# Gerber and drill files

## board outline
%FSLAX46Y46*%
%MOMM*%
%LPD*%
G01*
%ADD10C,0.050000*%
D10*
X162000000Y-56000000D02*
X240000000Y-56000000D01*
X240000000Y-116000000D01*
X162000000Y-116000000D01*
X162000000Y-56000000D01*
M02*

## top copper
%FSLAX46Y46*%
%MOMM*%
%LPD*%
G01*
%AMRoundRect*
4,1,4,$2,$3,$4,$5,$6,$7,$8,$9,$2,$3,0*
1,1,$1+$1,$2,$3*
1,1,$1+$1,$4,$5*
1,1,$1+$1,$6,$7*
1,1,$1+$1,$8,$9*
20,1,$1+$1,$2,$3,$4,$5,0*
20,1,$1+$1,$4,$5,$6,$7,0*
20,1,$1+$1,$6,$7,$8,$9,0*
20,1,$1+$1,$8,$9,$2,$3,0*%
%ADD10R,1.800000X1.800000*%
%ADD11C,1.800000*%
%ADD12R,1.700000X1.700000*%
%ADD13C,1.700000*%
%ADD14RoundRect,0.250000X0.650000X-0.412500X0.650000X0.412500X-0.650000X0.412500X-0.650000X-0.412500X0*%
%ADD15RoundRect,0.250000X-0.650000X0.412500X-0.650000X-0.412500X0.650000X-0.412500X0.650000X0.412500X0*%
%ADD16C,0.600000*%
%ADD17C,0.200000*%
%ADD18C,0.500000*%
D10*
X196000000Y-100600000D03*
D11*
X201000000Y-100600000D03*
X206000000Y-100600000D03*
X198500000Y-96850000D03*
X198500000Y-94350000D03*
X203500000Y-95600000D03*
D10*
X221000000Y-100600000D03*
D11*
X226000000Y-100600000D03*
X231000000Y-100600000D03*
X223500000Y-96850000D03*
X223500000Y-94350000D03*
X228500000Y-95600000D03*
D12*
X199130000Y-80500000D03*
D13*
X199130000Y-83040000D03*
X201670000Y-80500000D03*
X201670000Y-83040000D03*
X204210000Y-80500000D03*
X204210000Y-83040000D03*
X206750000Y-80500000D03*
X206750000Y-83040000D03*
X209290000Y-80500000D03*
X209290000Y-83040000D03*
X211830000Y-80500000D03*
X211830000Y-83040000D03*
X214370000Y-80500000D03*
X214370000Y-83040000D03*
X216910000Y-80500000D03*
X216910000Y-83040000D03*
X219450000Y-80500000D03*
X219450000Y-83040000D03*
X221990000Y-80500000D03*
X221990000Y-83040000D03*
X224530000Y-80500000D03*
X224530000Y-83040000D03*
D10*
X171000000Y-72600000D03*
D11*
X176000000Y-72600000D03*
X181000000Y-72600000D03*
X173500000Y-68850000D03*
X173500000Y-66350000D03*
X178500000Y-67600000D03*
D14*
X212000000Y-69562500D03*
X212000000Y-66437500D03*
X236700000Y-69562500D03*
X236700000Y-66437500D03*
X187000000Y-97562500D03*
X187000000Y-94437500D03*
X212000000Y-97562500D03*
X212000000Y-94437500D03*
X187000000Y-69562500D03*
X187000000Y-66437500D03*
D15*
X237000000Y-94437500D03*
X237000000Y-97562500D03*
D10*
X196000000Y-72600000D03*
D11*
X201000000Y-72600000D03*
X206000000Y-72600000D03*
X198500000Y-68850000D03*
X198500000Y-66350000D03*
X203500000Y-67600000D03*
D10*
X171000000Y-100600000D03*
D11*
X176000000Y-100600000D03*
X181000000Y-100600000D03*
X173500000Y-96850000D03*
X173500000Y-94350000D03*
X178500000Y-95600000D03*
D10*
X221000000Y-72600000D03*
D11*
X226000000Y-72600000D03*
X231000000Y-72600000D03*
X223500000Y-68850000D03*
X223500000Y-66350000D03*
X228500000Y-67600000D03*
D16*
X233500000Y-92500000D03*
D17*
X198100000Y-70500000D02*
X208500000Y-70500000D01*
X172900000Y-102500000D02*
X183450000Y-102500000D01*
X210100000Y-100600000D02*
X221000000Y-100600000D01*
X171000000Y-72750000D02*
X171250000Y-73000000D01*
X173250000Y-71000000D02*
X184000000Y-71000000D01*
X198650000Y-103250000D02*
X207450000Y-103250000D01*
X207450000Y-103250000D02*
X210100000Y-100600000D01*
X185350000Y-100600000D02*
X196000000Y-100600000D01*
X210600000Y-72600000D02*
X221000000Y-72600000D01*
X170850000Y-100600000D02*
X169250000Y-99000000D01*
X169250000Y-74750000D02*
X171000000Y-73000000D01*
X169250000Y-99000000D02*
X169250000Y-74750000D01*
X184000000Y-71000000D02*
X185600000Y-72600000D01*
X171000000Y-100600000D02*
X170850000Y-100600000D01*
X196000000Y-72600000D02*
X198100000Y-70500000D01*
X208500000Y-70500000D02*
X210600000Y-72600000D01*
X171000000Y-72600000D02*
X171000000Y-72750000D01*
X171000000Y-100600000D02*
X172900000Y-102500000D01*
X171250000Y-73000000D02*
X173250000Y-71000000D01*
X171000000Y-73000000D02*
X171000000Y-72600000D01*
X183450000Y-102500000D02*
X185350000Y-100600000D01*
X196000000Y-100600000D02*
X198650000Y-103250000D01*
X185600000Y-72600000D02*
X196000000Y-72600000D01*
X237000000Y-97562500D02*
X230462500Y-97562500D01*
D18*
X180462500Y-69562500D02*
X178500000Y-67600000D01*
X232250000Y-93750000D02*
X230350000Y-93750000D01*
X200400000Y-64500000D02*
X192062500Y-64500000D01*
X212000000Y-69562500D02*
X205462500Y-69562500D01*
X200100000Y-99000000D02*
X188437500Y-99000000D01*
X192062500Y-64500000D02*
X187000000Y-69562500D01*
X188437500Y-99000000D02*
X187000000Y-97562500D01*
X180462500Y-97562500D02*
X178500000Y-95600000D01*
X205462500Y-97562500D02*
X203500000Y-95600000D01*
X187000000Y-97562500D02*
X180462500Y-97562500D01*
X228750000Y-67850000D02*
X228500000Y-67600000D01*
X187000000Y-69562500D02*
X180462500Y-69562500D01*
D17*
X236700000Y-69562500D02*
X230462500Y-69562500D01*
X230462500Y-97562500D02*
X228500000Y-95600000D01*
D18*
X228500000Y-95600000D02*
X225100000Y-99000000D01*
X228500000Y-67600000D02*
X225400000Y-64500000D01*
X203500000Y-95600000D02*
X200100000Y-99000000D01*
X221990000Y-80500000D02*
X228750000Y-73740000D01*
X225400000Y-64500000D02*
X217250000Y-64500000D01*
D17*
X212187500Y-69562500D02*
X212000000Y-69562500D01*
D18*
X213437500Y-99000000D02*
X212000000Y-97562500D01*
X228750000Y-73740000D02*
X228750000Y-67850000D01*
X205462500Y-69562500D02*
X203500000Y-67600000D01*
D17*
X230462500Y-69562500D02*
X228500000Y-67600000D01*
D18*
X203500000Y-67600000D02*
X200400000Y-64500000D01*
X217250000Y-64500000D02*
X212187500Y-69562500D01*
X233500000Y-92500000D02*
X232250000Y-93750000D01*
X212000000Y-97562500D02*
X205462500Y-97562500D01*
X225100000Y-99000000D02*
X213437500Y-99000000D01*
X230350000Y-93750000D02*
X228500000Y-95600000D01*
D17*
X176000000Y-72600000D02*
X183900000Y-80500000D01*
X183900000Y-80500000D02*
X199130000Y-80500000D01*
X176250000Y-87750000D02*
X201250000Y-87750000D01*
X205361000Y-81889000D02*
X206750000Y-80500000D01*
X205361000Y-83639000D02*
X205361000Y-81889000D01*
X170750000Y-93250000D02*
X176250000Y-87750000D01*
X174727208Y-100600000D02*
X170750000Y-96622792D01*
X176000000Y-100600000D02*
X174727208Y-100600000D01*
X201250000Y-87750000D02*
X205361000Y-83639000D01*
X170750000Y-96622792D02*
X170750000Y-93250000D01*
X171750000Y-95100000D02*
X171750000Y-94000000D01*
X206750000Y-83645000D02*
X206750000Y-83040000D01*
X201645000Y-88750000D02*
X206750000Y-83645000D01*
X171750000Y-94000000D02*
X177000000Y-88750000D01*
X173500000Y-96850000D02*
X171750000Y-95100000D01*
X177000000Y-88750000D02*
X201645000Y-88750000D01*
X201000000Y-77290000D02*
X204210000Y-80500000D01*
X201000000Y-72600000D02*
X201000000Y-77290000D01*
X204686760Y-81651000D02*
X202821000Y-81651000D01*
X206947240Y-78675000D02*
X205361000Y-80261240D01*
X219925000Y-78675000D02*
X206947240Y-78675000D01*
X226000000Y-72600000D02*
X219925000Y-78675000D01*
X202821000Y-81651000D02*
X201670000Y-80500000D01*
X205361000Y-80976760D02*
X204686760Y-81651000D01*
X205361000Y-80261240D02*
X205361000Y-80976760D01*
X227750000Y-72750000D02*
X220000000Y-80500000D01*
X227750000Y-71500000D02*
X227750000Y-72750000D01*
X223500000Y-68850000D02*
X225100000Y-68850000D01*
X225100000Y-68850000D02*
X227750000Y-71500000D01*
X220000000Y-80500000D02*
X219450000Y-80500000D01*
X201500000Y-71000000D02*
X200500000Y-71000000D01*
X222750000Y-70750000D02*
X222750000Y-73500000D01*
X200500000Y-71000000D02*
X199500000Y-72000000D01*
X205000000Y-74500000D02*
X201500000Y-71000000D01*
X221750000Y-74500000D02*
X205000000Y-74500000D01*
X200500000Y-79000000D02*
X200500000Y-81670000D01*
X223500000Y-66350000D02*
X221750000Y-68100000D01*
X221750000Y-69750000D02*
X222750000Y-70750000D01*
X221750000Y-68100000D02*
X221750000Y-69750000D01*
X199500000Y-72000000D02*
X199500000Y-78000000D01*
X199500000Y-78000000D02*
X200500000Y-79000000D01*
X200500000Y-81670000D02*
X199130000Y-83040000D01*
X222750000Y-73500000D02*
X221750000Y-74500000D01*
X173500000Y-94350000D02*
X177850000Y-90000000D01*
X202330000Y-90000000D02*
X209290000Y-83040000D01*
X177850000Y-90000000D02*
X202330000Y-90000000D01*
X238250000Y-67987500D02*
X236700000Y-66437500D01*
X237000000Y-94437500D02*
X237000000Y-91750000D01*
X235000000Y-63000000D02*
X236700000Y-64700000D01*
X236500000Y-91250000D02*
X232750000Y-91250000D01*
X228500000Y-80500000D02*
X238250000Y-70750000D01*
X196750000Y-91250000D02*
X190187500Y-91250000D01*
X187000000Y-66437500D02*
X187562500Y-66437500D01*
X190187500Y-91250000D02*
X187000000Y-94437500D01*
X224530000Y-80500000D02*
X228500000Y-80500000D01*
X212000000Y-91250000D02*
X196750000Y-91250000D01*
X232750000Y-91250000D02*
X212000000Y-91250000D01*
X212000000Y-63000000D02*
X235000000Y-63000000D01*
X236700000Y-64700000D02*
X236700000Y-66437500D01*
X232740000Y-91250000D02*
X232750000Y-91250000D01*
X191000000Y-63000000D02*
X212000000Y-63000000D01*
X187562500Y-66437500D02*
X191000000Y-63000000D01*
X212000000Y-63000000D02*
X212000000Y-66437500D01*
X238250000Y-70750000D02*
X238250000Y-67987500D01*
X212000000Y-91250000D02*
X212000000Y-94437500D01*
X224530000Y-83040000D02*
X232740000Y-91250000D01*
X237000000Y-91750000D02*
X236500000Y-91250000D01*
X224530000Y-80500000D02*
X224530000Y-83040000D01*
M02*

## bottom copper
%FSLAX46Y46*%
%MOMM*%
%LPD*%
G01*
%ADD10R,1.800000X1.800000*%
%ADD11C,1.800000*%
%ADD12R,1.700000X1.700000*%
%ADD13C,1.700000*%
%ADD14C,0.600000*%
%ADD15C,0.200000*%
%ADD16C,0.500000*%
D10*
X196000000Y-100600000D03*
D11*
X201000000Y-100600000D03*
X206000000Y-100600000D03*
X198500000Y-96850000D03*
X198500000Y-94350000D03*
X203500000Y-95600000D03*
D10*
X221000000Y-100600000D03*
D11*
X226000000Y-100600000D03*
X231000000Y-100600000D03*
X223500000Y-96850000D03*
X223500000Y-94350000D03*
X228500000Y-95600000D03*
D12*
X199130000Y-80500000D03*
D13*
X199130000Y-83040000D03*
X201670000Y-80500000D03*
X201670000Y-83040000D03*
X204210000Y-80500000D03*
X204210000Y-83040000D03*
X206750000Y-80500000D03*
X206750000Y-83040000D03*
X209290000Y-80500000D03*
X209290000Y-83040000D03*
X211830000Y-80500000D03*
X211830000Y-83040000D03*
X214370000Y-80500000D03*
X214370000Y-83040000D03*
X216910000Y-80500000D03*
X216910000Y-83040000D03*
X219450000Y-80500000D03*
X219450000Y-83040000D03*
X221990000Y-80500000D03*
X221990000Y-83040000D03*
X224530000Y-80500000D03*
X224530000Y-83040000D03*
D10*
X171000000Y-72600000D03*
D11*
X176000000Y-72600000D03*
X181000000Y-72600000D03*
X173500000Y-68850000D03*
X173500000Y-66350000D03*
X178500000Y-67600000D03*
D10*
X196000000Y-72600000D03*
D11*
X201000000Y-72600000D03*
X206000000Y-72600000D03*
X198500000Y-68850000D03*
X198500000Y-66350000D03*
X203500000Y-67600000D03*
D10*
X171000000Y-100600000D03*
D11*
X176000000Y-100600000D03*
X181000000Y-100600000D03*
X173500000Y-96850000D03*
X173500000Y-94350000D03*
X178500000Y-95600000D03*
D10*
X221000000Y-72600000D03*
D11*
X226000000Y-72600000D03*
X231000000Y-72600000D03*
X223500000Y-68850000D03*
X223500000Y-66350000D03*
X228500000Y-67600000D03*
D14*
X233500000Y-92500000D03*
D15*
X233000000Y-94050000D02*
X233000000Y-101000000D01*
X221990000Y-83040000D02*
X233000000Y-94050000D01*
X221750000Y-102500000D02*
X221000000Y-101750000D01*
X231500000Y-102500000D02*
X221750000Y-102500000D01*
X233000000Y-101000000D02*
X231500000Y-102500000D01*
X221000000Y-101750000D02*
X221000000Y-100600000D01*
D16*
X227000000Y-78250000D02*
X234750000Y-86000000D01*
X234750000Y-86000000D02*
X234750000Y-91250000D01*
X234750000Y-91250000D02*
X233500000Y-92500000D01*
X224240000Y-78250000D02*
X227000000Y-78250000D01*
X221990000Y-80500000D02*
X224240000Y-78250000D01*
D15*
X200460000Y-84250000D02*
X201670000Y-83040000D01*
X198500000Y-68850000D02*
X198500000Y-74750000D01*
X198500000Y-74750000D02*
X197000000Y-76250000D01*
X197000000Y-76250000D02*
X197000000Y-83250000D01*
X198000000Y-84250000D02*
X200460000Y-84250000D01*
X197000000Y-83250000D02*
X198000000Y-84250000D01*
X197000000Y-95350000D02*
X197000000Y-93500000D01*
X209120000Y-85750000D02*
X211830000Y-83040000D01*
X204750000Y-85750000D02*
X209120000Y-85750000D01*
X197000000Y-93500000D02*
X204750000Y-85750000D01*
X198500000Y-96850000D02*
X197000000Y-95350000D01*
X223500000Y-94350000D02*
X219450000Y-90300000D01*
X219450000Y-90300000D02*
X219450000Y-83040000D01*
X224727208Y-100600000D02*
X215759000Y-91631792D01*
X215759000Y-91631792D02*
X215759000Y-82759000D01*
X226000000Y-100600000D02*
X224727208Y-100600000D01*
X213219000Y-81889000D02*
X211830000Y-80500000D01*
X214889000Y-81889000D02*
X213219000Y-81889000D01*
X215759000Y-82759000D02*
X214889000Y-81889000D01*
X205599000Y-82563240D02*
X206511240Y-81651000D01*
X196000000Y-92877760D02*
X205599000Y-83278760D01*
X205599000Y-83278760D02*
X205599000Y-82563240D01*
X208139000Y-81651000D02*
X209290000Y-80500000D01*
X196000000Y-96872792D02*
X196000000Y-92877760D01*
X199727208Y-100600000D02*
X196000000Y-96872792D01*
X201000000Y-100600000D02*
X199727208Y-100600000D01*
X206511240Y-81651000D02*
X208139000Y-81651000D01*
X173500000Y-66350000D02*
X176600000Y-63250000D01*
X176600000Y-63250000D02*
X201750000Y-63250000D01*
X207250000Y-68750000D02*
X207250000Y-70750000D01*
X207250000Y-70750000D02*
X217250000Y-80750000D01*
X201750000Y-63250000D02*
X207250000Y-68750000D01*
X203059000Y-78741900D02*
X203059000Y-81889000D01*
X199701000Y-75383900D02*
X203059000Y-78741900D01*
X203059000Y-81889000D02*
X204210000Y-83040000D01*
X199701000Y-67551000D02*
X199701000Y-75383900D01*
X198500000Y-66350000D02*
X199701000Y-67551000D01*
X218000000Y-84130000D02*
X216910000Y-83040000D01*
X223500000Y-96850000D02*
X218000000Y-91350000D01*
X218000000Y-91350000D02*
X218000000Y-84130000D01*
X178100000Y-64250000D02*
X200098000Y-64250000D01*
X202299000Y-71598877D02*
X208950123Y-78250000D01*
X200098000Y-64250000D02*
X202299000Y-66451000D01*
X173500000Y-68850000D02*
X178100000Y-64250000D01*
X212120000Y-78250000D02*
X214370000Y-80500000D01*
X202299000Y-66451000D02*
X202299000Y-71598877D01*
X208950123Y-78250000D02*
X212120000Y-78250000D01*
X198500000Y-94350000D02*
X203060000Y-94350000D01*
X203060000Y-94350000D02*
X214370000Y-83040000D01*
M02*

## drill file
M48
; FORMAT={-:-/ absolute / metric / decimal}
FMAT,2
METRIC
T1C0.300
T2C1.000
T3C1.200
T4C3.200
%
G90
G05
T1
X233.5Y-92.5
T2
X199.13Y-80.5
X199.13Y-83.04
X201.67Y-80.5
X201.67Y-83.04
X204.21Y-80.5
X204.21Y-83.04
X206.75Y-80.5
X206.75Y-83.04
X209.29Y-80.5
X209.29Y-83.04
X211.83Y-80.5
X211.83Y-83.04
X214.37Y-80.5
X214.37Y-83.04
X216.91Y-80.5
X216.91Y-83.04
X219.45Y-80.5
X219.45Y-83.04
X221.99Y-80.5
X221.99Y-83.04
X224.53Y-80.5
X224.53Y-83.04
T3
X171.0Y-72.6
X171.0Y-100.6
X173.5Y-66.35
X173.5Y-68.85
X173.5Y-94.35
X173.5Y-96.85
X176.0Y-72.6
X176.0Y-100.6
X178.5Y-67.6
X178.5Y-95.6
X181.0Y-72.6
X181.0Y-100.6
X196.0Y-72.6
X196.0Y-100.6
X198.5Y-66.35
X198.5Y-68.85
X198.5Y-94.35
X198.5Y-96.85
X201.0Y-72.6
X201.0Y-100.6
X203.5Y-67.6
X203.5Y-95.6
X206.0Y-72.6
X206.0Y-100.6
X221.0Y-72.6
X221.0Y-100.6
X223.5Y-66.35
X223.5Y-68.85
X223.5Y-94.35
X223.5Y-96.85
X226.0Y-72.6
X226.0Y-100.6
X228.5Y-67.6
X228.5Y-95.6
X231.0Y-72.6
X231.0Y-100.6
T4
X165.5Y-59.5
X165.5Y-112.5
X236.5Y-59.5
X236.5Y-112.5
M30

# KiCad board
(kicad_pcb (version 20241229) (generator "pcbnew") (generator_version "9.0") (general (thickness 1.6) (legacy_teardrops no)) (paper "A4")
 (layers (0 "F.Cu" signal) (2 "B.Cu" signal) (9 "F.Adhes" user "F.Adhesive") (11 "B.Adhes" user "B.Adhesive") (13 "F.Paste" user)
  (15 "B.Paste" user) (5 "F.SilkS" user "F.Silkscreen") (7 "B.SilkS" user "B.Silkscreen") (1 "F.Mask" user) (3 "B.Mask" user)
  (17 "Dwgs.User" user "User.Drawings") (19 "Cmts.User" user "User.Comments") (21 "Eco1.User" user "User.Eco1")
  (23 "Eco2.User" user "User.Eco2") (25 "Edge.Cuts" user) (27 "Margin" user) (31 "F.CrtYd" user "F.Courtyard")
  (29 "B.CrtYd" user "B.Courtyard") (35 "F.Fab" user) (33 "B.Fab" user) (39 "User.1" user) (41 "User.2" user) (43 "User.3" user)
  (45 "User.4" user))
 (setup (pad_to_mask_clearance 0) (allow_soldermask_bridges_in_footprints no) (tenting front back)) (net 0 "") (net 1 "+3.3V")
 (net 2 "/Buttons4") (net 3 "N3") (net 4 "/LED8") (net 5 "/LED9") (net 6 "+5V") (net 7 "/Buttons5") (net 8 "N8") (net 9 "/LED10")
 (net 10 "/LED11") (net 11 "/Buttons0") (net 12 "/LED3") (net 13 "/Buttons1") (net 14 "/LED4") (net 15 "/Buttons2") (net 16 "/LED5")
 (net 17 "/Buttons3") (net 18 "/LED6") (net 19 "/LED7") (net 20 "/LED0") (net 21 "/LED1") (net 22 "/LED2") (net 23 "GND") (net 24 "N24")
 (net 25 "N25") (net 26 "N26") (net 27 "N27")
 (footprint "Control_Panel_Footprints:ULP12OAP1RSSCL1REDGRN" (layer "F.Cu") (at 196 100.6)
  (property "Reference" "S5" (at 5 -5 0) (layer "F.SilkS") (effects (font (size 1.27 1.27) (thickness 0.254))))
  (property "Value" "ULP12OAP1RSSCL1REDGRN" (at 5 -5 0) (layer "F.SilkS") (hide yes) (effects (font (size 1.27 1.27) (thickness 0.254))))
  (pad "1" thru_hole rect (at 0 0) (size 1.8 1.8) (drill 1.2) (layers "*.Cu" "*.Mask") (remove_unused_layers no) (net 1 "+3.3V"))
  (pad "2" thru_hole circle (at 5 0) (size 1.8 1.8) (drill 1.2) (layers "*.Cu" "*.Mask") (remove_unused_layers no) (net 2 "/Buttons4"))
  (pad "3" thru_hole circle (at 10 0) (size 1.8 1.8) (drill 1.2) (layers "*.Cu" "*.Mask") (remove_unused_layers no) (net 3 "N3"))
  (pad "L1" thru_hole circle (at 2.5 -3.75) (size 1.8 1.8) (drill 1.2) (layers "*.Cu" "*.Mask") (remove_unused_layers no) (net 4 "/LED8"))
  (pad "L2" thru_hole circle (at 2.5 -6.25) (size 1.8 1.8) (drill 1.2) (layers "*.Cu" "*.Mask") (remove_unused_layers no) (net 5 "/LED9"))
  (pad "LC1" thru_hole circle (at 7.5 -5) (size 1.8 1.8) (drill 1.2) (layers "*.Cu" "*.Mask") (remove_unused_layers no) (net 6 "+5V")))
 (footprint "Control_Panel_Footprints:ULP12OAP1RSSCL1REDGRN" (layer "F.Cu") (at 221 100.6)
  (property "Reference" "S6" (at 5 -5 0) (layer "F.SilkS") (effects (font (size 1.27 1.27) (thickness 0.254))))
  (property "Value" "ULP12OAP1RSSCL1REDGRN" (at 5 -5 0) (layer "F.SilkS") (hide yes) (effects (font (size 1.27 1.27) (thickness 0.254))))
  (pad "1" thru_hole rect (at 0 0) (size 1.8 1.8) (drill 1.2) (layers "*.Cu" "*.Mask") (remove_unused_layers no) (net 1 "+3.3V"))
  (pad "2" thru_hole circle (at 5 0) (size 1.8 1.8) (drill 1.2) (layers "*.Cu" "*.Mask") (remove_unused_layers no) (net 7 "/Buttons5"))
  (pad "3" thru_hole circle (at 10 0) (size 1.8 1.8) (drill 1.2) (layers "*.Cu" "*.Mask") (remove_unused_layers no) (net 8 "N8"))
  (pad "L1" thru_hole circle (at 2.5 -3.75) (size 1.8 1.8) (drill 1.2) (layers "*.Cu" "*.Mask") (remove_unused_layers no) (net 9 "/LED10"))
  (pad "L2" thru_hole circle (at 2.5 -6.25) (size 1.8 1.8) (drill 1.2) (layers "*.Cu" "*.Mask") (remove_unused_layers no) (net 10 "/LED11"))
  (pad "LC1" thru_hole circle (at 7.5 -5) (size 1.8 1.8) (drill 1.2) (layers "*.Cu" "*.Mask") (remove_unused_layers no) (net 6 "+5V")))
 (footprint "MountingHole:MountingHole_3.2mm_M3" (layer "F.Cu") (at 165.5 59.5)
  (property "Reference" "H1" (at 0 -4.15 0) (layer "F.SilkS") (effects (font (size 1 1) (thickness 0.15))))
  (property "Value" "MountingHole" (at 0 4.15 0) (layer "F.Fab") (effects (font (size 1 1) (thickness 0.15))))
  (pad "" np_thru_hole circle (at 0 0) (size 3.2 3.2) (drill 3.2) (layers "*.Cu" "*.Mask")))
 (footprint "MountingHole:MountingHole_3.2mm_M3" (layer "F.Cu") (at 236.5 59.5)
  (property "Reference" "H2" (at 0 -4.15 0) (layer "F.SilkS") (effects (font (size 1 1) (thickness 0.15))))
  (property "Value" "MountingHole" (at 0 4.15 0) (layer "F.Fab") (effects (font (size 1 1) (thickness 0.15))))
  (pad "" np_thru_hole circle (at 0 0) (size 3.2 3.2) (drill 3.2) (layers "*.Cu" "*.Mask")))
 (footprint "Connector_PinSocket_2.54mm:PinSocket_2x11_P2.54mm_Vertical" (layer "F.Cu") (at 199.13 80.5 90)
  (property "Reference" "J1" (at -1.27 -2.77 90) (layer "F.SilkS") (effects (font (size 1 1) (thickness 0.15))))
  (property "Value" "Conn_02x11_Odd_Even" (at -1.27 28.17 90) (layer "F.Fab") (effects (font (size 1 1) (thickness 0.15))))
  (pad "1" thru_hole rect (at 0 0 90) (size 1.7 1.7) (drill 1) (layers "*.Cu" "*.Mask") (remove_unused_layers no) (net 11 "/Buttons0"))
  (pad "2" thru_hole circle (at -2.54 0 90) (size 1.7 1.7) (drill 1) (layers "*.Cu" "*.Mask") (remove_unused_layers no) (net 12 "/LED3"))
  (pad "3" thru_hole circle (at 0 2.54 90) (size 1.7 1.7) (drill 1) (layers "*.Cu" "*.Mask") (remove_unused_layers no) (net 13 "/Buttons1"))
  (pad "4" thru_hole circle (at -2.54 2.54 90) (size 1.7 1.7) (drill 1) (layers "*.Cu" "*.Mask") (remove_unused_layers no) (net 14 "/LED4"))
  (pad "5" thru_hole circle (at 0 5.08 90) (size 1.7 1.7) (drill 1) (layers "*.Cu" "*.Mask") (remove_unused_layers no) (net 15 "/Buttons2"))
  (pad "6" thru_hole circle (at -2.54 5.08 90) (size 1.7 1.7) (drill 1) (layers "*.Cu" "*.Mask") (remove_unused_layers no) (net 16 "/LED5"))
  (pad "7" thru_hole circle (at 0 7.62 90) (size 1.7 1.7) (drill 1) (layers "*.Cu" "*.Mask") (remove_unused_layers no) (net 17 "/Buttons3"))
  (pad "8" thru_hole circle (at -2.54 7.62 90) (size 1.7 1.7) (drill 1) (layers "*.Cu" "*.Mask") (remove_unused_layers no) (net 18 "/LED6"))
  (pad "9" thru_hole circle (at 0 10.16 90) (size 1.7 1.7) (drill 1) (layers "*.Cu" "*.Mask") (remove_unused_layers no) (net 2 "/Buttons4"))
  (pad "10" thru_hole circle (at -2.54 10.16 90) (size 1.7 1.7) (drill 1) (layers "*.Cu" "*.Mask") (remove_unused_layers no)
   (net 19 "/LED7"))
  (pad "11" thru_hole circle (at 0 12.7 90) (size 1.7 1.7) (drill 1) (layers "*.Cu" "*.Mask") (remove_unused_layers no) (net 7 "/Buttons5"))
  (pad "12" thru_hole circle (at -2.54 12.7 90) (size 1.7 1.7) (drill 1) (layers "*.Cu" "*.Mask") (remove_unused_layers no) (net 4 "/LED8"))
  (pad "13" thru_hole circle (at 0 15.24 90) (size 1.7 1.7) (drill 1) (layers "*.Cu" "*.Mask") (remove_unused_layers no) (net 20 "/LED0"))
  (pad "14" thru_hole circle (at -2.54 15.24 90) (size 1.7 1.7) (drill 1) (layers "*.Cu" "*.Mask") (remove_unused_layers no) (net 5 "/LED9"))
  (pad "15" thru_hole circle (at 0 17.78 90) (size 1.7 1.7) (drill 1) (layers "*.Cu" "*.Mask") (remove_unused_layers no) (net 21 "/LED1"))
  (pad "16" thru_hole circle (at -2.54 17.78 90) (size 1.7 1.7) (drill 1) (layers "*.Cu" "*.Mask") (remove_unused_layers no)
   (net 9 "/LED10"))
  (pad "17" thru_hole circle (at 0 20.32 90) (size 1.7 1.7) (drill 1) (layers "*.Cu" "*.Mask") (remove_unused_layers no) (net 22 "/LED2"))
  (pad "18" thru_hole circle (at -2.54 20.32 90) (size 1.7 1.7) (drill 1) (layers "*.Cu" "*.Mask") (remove_unused_layers no)
   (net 10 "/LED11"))
  (pad "19" thru_hole circle (at 0 22.86 90) (size 1.7 1.7) (drill 1) (layers "*.Cu" "*.Mask") (remove_unused_layers no) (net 6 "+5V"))
  (pad "20" thru_hole circle (at -2.54 22.86 90) (size 1.7 1.7) (drill 1) (layers "*.Cu" "*.Mask") (remove_unused_layers no) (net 1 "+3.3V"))
  (pad "21" thru_hole circle (at 0 25.4 90) (size 1.7 1.7) (drill 1) (layers "*.Cu" "*.Mask") (remove_unused_layers no) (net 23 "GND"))
  (pad "22" thru_hole circle (at -2.54 25.4 90) (size 1.7 1.7) (drill 1) (layers "*.Cu" "*.Mask") (remove_unused_layers no) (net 23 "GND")))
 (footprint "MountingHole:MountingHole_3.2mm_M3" (layer "F.Cu") (at 236.5 112.5)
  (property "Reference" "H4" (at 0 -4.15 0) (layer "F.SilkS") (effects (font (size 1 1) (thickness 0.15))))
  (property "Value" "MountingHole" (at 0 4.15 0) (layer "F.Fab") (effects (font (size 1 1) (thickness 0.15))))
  (pad "" np_thru_hole circle (at 0 0) (size 3.2 3.2) (drill 3.2) (layers "*.Cu" "*.Mask")))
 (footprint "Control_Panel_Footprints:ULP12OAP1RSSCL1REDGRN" (layer "F.Cu") (at 171 72.6)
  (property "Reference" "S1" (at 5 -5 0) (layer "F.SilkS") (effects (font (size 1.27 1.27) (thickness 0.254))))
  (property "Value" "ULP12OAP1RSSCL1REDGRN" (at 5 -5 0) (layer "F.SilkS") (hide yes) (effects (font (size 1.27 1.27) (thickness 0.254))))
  (pad "1" thru_hole rect (at 0 0) (size 1.8 1.8) (drill 1.2) (layers "*.Cu" "*.Mask") (remove_unused_layers no) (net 1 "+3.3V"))
  (pad "2" thru_hole circle (at 5 0) (size 1.8 1.8) (drill 1.2) (layers "*.Cu" "*.Mask") (remove_unused_layers no) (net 11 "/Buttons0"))
  (pad "3" thru_hole circle (at 10 0) (size 1.8 1.8) (drill 1.2) (layers "*.Cu" "*.Mask") (remove_unused_layers no) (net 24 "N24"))
  (pad "L1" thru_hole circle (at 2.5 -3.75) (size 1.8 1.8) (drill 1.2) (layers "*.Cu" "*.Mask") (remove_unused_layers no) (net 20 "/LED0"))
  (pad "L2" thru_hole circle (at 2.5 -6.25) (size 1.8 1.8) (drill 1.2) (layers "*.Cu" "*.Mask") (remove_unused_layers no) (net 21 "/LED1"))
  (pad "LC1" thru_hole circle (at 7.5 -5) (size 1.8 1.8) (drill 1.2) (layers "*.Cu" "*.Mask") (remove_unused_layers no) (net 6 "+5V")))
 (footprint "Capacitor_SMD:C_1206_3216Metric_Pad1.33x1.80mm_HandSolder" (layer "F.Cu") (at 212 68 90)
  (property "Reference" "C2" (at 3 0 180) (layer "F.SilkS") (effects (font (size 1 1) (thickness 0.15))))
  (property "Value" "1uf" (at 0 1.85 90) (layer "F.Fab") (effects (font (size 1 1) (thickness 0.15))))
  (pad "1" smd roundrect (at -1.5625 0 90) (size 1.325 1.8) (layers "F.Cu" "F.Mask" "F.Paste") (roundrect_rratio 0.188679) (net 6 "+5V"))
  (pad "2" smd roundrect (at 1.5625 0 90) (size 1.325 1.8) (layers "F.Cu" "F.Mask" "F.Paste") (roundrect_rratio 0.188679) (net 23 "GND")))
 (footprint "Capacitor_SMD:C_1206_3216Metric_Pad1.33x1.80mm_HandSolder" (layer "F.Cu") (at 236.7 68 90)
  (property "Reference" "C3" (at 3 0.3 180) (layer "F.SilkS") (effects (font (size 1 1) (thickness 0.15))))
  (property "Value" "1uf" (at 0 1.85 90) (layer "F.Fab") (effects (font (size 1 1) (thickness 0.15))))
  (pad "1" smd roundrect (at -1.5625 0 90) (size 1.325 1.8) (layers "F.Cu" "F.Mask" "F.Paste") (roundrect_rratio 0.188679) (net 6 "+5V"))
  (pad "2" smd roundrect (at 1.5625 0 90) (size 1.325 1.8) (layers "F.Cu" "F.Mask" "F.Paste") (roundrect_rratio 0.188679) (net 23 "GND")))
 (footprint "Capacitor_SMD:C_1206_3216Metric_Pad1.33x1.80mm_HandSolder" (layer "F.Cu") (at 187 96 90)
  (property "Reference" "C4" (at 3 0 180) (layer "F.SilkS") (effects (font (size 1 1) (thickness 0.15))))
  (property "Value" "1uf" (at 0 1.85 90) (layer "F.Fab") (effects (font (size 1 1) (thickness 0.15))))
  (pad "1" smd roundrect (at -1.5625 0 90) (size 1.325 1.8) (layers "F.Cu" "F.Mask" "F.Paste") (roundrect_rratio 0.188679) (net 6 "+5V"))
  (pad "2" smd roundrect (at 1.5625 0 90) (size 1.325 1.8) (layers "F.Cu" "F.Mask" "F.Paste") (roundrect_rratio 0.188679) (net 23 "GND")))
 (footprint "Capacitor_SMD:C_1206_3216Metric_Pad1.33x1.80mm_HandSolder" (layer "F.Cu") (at 212 96 90)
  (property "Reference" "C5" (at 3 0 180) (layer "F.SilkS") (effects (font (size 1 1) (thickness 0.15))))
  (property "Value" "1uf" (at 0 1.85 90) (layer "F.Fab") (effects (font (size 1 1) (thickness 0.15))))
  (pad "1" smd roundrect (at -1.5625 0 90) (size 1.325 1.8) (layers "F.Cu" "F.Mask" "F.Paste") (roundrect_rratio 0.188679) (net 6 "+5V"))
  (pad "2" smd roundrect (at 1.5625 0 90) (size 1.325 1.8) (layers "F.Cu" "F.Mask" "F.Paste") (roundrect_rratio 0.188679) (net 23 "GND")))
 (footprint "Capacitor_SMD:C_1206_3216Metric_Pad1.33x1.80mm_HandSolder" (layer "F.Cu") (at 187 68 90)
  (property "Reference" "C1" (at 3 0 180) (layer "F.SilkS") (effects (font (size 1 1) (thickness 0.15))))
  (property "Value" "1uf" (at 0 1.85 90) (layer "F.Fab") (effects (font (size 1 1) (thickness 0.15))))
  (pad "1" smd roundrect (at -1.5625 0 90) (size 1.325 1.8) (layers "F.Cu" "F.Mask" "F.Paste") (roundrect_rratio 0.188679) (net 6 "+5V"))
  (pad "2" smd roundrect (at 1.5625 0 90) (size 1.325 1.8) (layers "F.Cu" "F.Mask" "F.Paste") (roundrect_rratio 0.188679) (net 23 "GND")))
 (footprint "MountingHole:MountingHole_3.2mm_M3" (layer "F.Cu") (at 165.5 112.5)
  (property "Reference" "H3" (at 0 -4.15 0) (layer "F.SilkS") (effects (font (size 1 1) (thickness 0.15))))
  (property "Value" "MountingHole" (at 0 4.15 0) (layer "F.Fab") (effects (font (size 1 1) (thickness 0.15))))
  (pad "" np_thru_hole circle (at 0 0) (size 3.2 3.2) (drill 3.2) (layers "*.Cu" "*.Mask")))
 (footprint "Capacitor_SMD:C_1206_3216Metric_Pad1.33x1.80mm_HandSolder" (layer "F.Cu") (at 237 96 -90)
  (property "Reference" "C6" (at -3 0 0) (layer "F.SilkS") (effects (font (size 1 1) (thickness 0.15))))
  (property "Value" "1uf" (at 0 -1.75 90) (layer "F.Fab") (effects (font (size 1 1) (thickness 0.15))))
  (pad "1" smd roundrect (at -1.5625 0 270) (size 1.325 1.8) (layers "F.Cu" "F.Mask" "F.Paste") (roundrect_rratio 0.188679) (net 23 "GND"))
  (pad "2" smd roundrect (at 1.5625 0 270) (size 1.325 1.8) (layers "F.Cu" "F.Mask" "F.Paste") (roundrect_rratio 0.188679) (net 6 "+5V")))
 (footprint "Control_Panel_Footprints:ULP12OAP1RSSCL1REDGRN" (layer "F.Cu") (at 196 72.6)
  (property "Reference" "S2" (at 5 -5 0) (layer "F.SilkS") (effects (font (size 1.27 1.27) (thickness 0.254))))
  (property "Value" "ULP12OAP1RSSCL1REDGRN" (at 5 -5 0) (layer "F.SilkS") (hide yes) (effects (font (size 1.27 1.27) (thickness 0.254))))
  (pad "1" thru_hole rect (at 0 0) (size 1.8 1.8) (drill 1.2) (layers "*.Cu" "*.Mask") (remove_unused_layers no) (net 1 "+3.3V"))
  (pad "2" thru_hole circle (at 5 0) (size 1.8 1.8) (drill 1.2) (layers "*.Cu" "*.Mask") (remove_unused_layers no) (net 15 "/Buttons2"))
  (pad "3" thru_hole circle (at 10 0) (size 1.8 1.8) (drill 1.2) (layers "*.Cu" "*.Mask") (remove_unused_layers no) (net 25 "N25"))
  (pad "L1" thru_hole circle (at 2.5 -3.75) (size 1.8 1.8) (drill 1.2) (layers "*.Cu" "*.Mask") (remove_unused_layers no) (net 14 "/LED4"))
  (pad "L2" thru_hole circle (at 2.5 -6.25) (size 1.8 1.8) (drill 1.2) (layers "*.Cu" "*.Mask") (remove_unused_layers no) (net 16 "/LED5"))
  (pad "LC1" thru_hole circle (at 7.5 -5) (size 1.8 1.8) (drill 1.2) (layers "*.Cu" "*.Mask") (remove_unused_layers no) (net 6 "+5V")))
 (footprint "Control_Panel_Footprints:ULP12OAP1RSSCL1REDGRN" (layer "F.Cu") (at 171 100.6)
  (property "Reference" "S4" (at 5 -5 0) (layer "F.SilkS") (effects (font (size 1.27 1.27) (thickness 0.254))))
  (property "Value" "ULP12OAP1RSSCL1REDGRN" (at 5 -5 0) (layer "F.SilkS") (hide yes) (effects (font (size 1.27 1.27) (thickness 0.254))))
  (pad "1" thru_hole rect (at 0 0) (size 1.8 1.8) (drill 1.2) (layers "*.Cu" "*.Mask") (remove_unused_layers no) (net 1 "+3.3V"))
  (pad "2" thru_hole circle (at 5 0) (size 1.8 1.8) (drill 1.2) (layers "*.Cu" "*.Mask") (remove_unused_layers no) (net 17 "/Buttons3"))
  (pad "3" thru_hole circle (at 10 0) (size 1.8 1.8) (drill 1.2) (layers "*.Cu" "*.Mask") (remove_unused_layers no) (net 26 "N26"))
  (pad "L1" thru_hole circle (at 2.5 -3.75) (size 1.8 1.8) (drill 1.2) (layers "*.Cu" "*.Mask") (remove_unused_layers no) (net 18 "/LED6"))
  (pad "L2" thru_hole circle (at 2.5 -6.25) (size 1.8 1.8) (drill 1.2) (layers "*.Cu" "*.Mask") (remove_unused_layers no) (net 19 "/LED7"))
  (pad "LC1" thru_hole circle (at 7.5 -5) (size 1.8 1.8) (drill 1.2) (layers "*.Cu" "*.Mask") (remove_unused_layers no) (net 6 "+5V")))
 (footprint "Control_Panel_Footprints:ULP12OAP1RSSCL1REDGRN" (layer "F.Cu") (at 221 72.6)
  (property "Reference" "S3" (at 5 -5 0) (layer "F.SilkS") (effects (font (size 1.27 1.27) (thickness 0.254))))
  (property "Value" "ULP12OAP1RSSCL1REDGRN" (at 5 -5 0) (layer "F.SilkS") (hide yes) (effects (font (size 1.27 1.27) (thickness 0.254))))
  (pad "1" thru_hole rect (at 0 0) (size 1.8 1.8) (drill 1.2) (layers "*.Cu" "*.Mask") (remove_unused_layers no) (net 1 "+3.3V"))
  (pad "2" thru_hole circle (at 5 0) (size 1.8 1.8) (drill 1.2) (layers "*.Cu" "*.Mask") (remove_unused_layers no) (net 13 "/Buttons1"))
  (pad "3" thru_hole circle (at 10 0) (size 1.8 1.8) (drill 1.2) (layers "*.Cu" "*.Mask") (remove_unused_layers no) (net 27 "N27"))
  (pad "L1" thru_hole circle (at 2.5 -3.75) (size 1.8 1.8) (drill 1.2) (layers "*.Cu" "*.Mask") (remove_unused_layers no) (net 22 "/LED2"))
  (pad "L2" thru_hole circle (at 2.5 -6.25) (size 1.8 1.8) (drill 1.2) (layers "*.Cu" "*.Mask") (remove_unused_layers no) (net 12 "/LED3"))
  (pad "LC1" thru_hole circle (at 7.5 -5) (size 1.8 1.8) (drill 1.2) (layers "*.Cu" "*.Mask") (remove_unused_layers no) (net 6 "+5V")))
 (gr_rect (start 162 56) (end 240 116) (stroke (width 0.05) (type solid)) (fill no) (layer "Edge.Cuts"))
 (segment (start 198.1 70.5) (end 208.5 70.5) (width 0.2) (layer "F.Cu") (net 1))
 (segment (start 172.9 102.5) (end 183.45 102.5) (width 0.2) (layer "F.Cu") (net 1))
 (segment (start 210.1 100.6) (end 221 100.6) (width 0.2) (layer "F.Cu") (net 1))
 (segment (start 171 72.75) (end 171.25 73) (width 0.2) (layer "F.Cu") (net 1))
 (segment (start 173.25 71) (end 184 71) (width 0.2) (layer "F.Cu") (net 1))
 (segment (start 198.65 103.25) (end 207.45 103.25) (width 0.2) (layer "F.Cu") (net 1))
 (segment (start 207.45 103.25) (end 210.1 100.6) (width 0.2) (layer "F.Cu") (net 1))
 (segment (start 185.35 100.6) (end 196 100.6) (width 0.2) (layer "F.Cu") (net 1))
 (segment (start 210.6 72.6) (end 221 72.6) (width 0.2) (layer "F.Cu") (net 1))
 (segment (start 170.85 100.6) (end 169.25 99) (width 0.2) (layer "F.Cu") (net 1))
 (segment (start 169.25 74.75) (end 171 73) (width 0.2) (layer "F.Cu") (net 1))
 (segment (start 169.25 99) (end 169.25 74.75) (width 0.2) (layer "F.Cu") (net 1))
 (segment (start 184 71) (end 185.6 72.6) (width 0.2) (layer "F.Cu") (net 1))
 (segment (start 171 100.6) (end 170.85 100.6) (width 0.2) (layer "F.Cu") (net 1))
 (segment (start 196 72.6) (end 198.1 70.5) (width 0.2) (layer "F.Cu") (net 1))
 (segment (start 208.5 70.5) (end 210.6 72.6) (width 0.2) (layer "F.Cu") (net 1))
 (segment (start 171 72.6) (end 171 72.75) (width 0.2) (layer "F.Cu") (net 1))
 (segment (start 171 100.6) (end 172.9 102.5) (width 0.2) (layer "F.Cu") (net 1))
 (segment (start 171.25 73) (end 173.25 71) (width 0.2) (layer "F.Cu") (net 1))
 (segment (start 171 73) (end 171 72.6) (width 0.2) (layer "F.Cu") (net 1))
 (segment (start 183.45 102.5) (end 185.35 100.6) (width 0.2) (layer "F.Cu") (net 1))
 (segment (start 196 100.6) (end 198.65 103.25) (width 0.2) (layer "F.Cu") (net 1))
 (segment (start 185.6 72.6) (end 196 72.6) (width 0.2) (layer "F.Cu") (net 1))
 (segment (start 233 94.05) (end 233 101) (width 0.2) (layer "B.Cu") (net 1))
 (segment (start 221.99 83.04) (end 233 94.05) (width 0.2) (layer "B.Cu") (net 1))
 (segment (start 221.75 102.5) (end 221 101.75) (width 0.2) (layer "B.Cu") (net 1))
 (segment (start 231.5 102.5) (end 221.75 102.5) (width 0.2) (layer "B.Cu") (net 1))
 (segment (start 233 101) (end 231.5 102.5) (width 0.2) (layer "B.Cu") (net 1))
 (segment (start 221 101.75) (end 221 100.6) (width 0.2) (layer "B.Cu") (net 1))
 (segment (start 237 97.5625) (end 230.4625 97.5625) (width 0.2) (layer "F.Cu") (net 6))
 (segment (start 180.4625 69.5625) (end 178.5 67.6) (width 0.5) (layer "F.Cu") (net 6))
 (segment (start 232.25 93.75) (end 230.35 93.75) (width 0.5) (layer "F.Cu") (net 6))
 (segment (start 200.4 64.5) (end 192.0625 64.5) (width 0.5) (layer "F.Cu") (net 6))
 (segment (start 212 69.5625) (end 205.4625 69.5625) (width 0.5) (layer "F.Cu") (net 6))
 (segment (start 200.1 99) (end 188.4375 99) (width 0.5) (layer "F.Cu") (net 6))
 (segment (start 192.0625 64.5) (end 187 69.5625) (width 0.5) (layer "F.Cu") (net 6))
 (segment (start 188.4375 99) (end 187 97.5625) (width 0.5) (layer "F.Cu") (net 6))
 (segment (start 180.4625 97.5625) (end 178.5 95.6) (width 0.5) (layer "F.Cu") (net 6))
 (segment (start 205.4625 97.5625) (end 203.5 95.6) (width 0.5) (layer "F.Cu") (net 6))
 (segment (start 187 97.5625) (end 180.4625 97.5625) (width 0.5) (layer "F.Cu") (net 6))
 (segment (start 228.75 67.85) (end 228.5 67.6) (width 0.5) (layer "F.Cu") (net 6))
 (segment (start 187 69.5625) (end 180.4625 69.5625) (width 0.5) (layer "F.Cu") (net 6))
 (segment (start 236.7 69.5625) (end 230.4625 69.5625) (width 0.2) (layer "F.Cu") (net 6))
 (segment (start 230.4625 97.5625) (end 228.5 95.6) (width 0.2) (layer "F.Cu") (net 6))
 (segment (start 228.5 95.6) (end 225.1 99) (width 0.5) (layer "F.Cu") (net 6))
 (segment (start 228.5 67.6) (end 225.4 64.5) (width 0.5) (layer "F.Cu") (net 6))
 (segment (start 203.5 95.6) (end 200.1 99) (width 0.5) (layer "F.Cu") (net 6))
 (segment (start 221.99 80.5) (end 228.75 73.74) (width 0.5) (layer "F.Cu") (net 6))
 (segment (start 225.4 64.5) (end 217.25 64.5) (width 0.5) (layer "F.Cu") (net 6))
 (segment (start 212.1875 69.5625) (end 212 69.5625) (width 0.2) (layer "F.Cu") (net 6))
 (segment (start 213.4375 99) (end 212 97.5625) (width 0.5) (layer "F.Cu") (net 6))
 (segment (start 228.75 73.74) (end 228.75 67.85) (width 0.5) (layer "F.Cu") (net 6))
 (segment (start 205.4625 69.5625) (end 203.5 67.6) (width 0.5) (layer "F.Cu") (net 6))
 (segment (start 230.4625 69.5625) (end 228.5 67.6) (width 0.2) (layer "F.Cu") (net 6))
 (segment (start 203.5 67.6) (end 200.4 64.5) (width 0.5) (layer "F.Cu") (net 6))
 (segment (start 217.25 64.5) (end 212.1875 69.5625) (width 0.5) (layer "F.Cu") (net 6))
 (segment (start 233.5 92.5) (end 232.25 93.75) (width 0.5) (layer "F.Cu") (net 6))
 (segment (start 212 97.5625) (end 205.4625 97.5625) (width 0.5) (layer "F.Cu") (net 6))
 (segment (start 225.1 99) (end 213.4375 99) (width 0.5) (layer "F.Cu") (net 6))
 (segment (start 230.35 93.75) (end 228.5 95.6) (width 0.5) (layer "F.Cu") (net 6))
 (via (at 233.5 92.5) (size 0.6) (drill 0.3) (layers "F.Cu" "B.Cu") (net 6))
 (segment (start 227 78.25) (end 234.75 86) (width 0.5) (layer "B.Cu") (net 6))
 (segment (start 234.75 86) (end 234.75 91.25) (width 0.5) (layer "B.Cu") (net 6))
 (segment (start 234.75 91.25) (end 233.5 92.5) (width 0.5) (layer "B.Cu") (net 6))
 (segment (start 224.24 78.25) (end 227 78.25) (width 0.5) (layer "B.Cu") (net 6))
 (segment (start 221.99 80.5) (end 224.24 78.25) (width 0.5) (layer "B.Cu") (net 6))
 (segment (start 200.46 84.25) (end 201.67 83.04) (width 0.2) (layer "B.Cu") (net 14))
 (segment (start 198.5 68.85) (end 198.5 74.75) (width 0.2) (layer "B.Cu") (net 14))
 (segment (start 198.5 74.75) (end 197 76.25) (width 0.2) (layer "B.Cu") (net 14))
 (segment (start 197 76.25) (end 197 83.25) (width 0.2) (layer "B.Cu") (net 14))
 (segment (start 198 84.25) (end 200.46 84.25) (width 0.2) (layer "B.Cu") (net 14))
 (segment (start 197 83.25) (end 198 84.25) (width 0.2) (layer "B.Cu") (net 14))
 (segment (start 197 95.35) (end 197 93.5) (width 0.2) (layer "B.Cu") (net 4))
 (segment (start 209.12 85.75) (end 211.83 83.04) (width 0.2) (layer "B.Cu") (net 4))
 (segment (start 204.75 85.75) (end 209.12 85.75) (width 0.2) (layer "B.Cu") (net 4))
 (segment (start 197 93.5) (end 204.75 85.75) (width 0.2) (layer "B.Cu") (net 4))
 (segment (start 198.5 96.85) (end 197 95.35) (width 0.2) (layer "B.Cu") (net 4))
 (segment (start 176 72.6) (end 183.9 80.5) (width 0.2) (layer "F.Cu") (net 11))
 (segment (start 183.9 80.5) (end 199.13 80.5) (width 0.2) (layer "F.Cu") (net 11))
 (segment (start 176.25 87.75) (end 201.25 87.75) (width 0.2) (layer "F.Cu") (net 17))
 (segment (start 205.361 81.889) (end 206.75 80.5) (width 0.2) (layer "F.Cu") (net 17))
 (segment (start 205.361 83.639) (end 205.361 81.889) (width 0.2) (layer "F.Cu") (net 17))
 (segment (start 170.75 93.25) (end 176.25 87.75) (width 0.2) (layer "F.Cu") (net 17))
 (segment (start 174.727208 100.6) (end 170.75 96.622792) (width 0.2) (layer "F.Cu") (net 17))
 (segment (start 176 100.6) (end 174.727208 100.6) (width 0.2) (layer "F.Cu") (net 17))
 (segment (start 201.25 87.75) (end 205.361 83.639) (width 0.2) (layer "F.Cu") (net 17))
 (segment (start 170.75 96.622792) (end 170.75 93.25) (width 0.2) (layer "F.Cu") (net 17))
 (segment (start 223.5 94.35) (end 219.45 90.3) (width 0.2) (layer "B.Cu") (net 10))
 (segment (start 219.45 90.3) (end 219.45 83.04) (width 0.2) (layer "B.Cu") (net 10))
 (segment (start 171.75 95.1) (end 171.75 94) (width 0.2) (layer "F.Cu") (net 18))
 (segment (start 206.75 83.645) (end 206.75 83.04) (width 0.2) (layer "F.Cu") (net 18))
 (segment (start 201.645 88.75) (end 206.75 83.645) (width 0.2) (layer "F.Cu") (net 18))
 (segment (start 171.75 94) (end 177 88.75) (width 0.2) (layer "F.Cu") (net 18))
 (segment (start 173.5 96.85) (end 171.75 95.1) (width 0.2) (layer "F.Cu") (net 18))
 (segment (start 177 88.75) (end 201.645 88.75) (width 0.2) (layer "F.Cu") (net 18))
 (segment (start 201 77.29) (end 204.21 80.5) (width 0.2) (layer "F.Cu") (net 15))
 (segment (start 201 72.6) (end 201 77.29) (width 0.2) (layer "F.Cu") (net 15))
 (segment (start 204.68676 81.651) (end 202.821 81.651) (width 0.2) (layer "F.Cu") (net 13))
 (segment (start 206.94724 78.675) (end 205.361 80.26124) (width 0.2) (layer "F.Cu") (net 13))
 (segment (start 219.925 78.675) (end 206.94724 78.675) (width 0.2) (layer "F.Cu") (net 13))
 (segment (start 226 72.6) (end 219.925 78.675) (width 0.2) (layer "F.Cu") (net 13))
 (segment (start 202.821 81.651) (end 201.67 80.5) (width 0.2) (layer "F.Cu") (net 13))
 (segment (start 205.361 80.97676) (end 204.68676 81.651) (width 0.2) (layer "F.Cu") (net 13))
 (segment (start 205.361 80.26124) (end 205.361 80.97676) (width 0.2) (layer "F.Cu") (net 13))
 (segment (start 227.75 72.75) (end 220 80.5) (width 0.2) (layer "F.Cu") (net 22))
 (segment (start 227.75 71.5) (end 227.75 72.75) (width 0.2) (layer "F.Cu") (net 22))
 (segment (start 223.5 68.85) (end 225.1 68.85) (width 0.2) (layer "F.Cu") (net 22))
 (segment (start 225.1 68.85) (end 227.75 71.5) (width 0.2) (layer "F.Cu") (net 22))
 (segment (start 220 80.5) (end 219.45 80.5) (width 0.2) (layer "F.Cu") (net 22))
 (segment (start 201.5 71) (end 200.5 71) (width 0.2) (layer "F.Cu") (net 12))
 (segment (start 222.75 70.75) (end 222.75 73.5) (width 0.2) (layer "F.Cu") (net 12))
 (segment (start 200.5 71) (end 199.5 72) (width 0.2) (layer "F.Cu") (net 12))
 (segment (start 205 74.5) (end 201.5 71) (width 0.2) (layer "F.Cu") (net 12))
 (segment (start 221.75 74.5) (end 205 74.5) (width 0.2) (layer "F.Cu") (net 12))
 (segment (start 200.5 79) (end 200.5 81.67) (width 0.2) (layer "F.Cu") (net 12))
 (segment (start 223.5 66.35) (end 221.75 68.1) (width 0.2) (layer "F.Cu") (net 12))
 (segment (start 221.75 69.75) (end 222.75 70.75) (width 0.2) (layer "F.Cu") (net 12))
 (segment (start 221.75 68.1) (end 221.75 69.75) (width 0.2) (layer "F.Cu") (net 12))
 (segment (start 199.5 72) (end 199.5 78) (width 0.2) (layer "F.Cu") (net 12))
 (segment (start 199.5 78) (end 200.5 79) (width 0.2) (layer "F.Cu") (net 12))
 (segment (start 200.5 81.67) (end 199.13 83.04) (width 0.2) (layer "F.Cu") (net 12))
 (segment (start 222.75 73.5) (end 221.75 74.5) (width 0.2) (layer "F.Cu") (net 12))
 (segment (start 224.727208 100.6) (end 215.759 91.631792) (width 0.2) (layer "B.Cu") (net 7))
 (segment (start 215.759 91.631792) (end 215.759 82.759) (width 0.2) (layer "B.Cu") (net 7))
 (segment (start 226 100.6) (end 224.727208 100.6) (width 0.2) (layer "B.Cu") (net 7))
 (segment (start 213.219 81.889) (end 211.83 80.5) (width 0.2) (layer "B.Cu") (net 7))
 (segment (start 214.889 81.889) (end 213.219 81.889) (width 0.2) (layer "B.Cu") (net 7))
 (segment (start 215.759 82.759) (end 214.889 81.889) (width 0.2) (layer "B.Cu") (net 7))
 (segment (start 205.599 82.56324) (end 206.51124 81.651) (width 0.2) (layer "B.Cu") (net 2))
 (segment (start 196 92.87776) (end 205.599 83.27876) (width 0.2) (layer "B.Cu") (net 2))
 (segment (start 205.599 83.27876) (end 205.599 82.56324) (width 0.2) (layer "B.Cu") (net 2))
 (segment (start 208.139 81.651) (end 209.29 80.5) (width 0.2) (layer "B.Cu") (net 2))
 (segment (start 196 96.872792) (end 196 92.87776) (width 0.2) (layer "B.Cu") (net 2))
 (segment (start 199.727208 100.6) (end 196 96.872792) (width 0.2) (layer "B.Cu") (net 2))
 (segment (start 201 100.6) (end 199.727208 100.6) (width 0.2) (layer "B.Cu") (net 2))
 (segment (start 206.51124 81.651) (end 208.139 81.651) (width 0.2) (layer "B.Cu") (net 2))
 (segment (start 173.5 66.35) (end 176.6 63.25) (width 0.2) (layer "B.Cu") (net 21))
 (segment (start 176.6 63.25) (end 201.75 63.25) (width 0.2) (layer "B.Cu") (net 21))
 (segment (start 207.25 68.75) (end 207.25 70.75) (width 0.2) (layer "B.Cu") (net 21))
 (segment (start 207.25 70.75) (end 217.25 80.75) (width 0.2) (layer "B.Cu") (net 21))
 (segment (start 201.75 63.25) (end 207.25 68.75) (width 0.2) (layer "B.Cu") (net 21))
 (segment (start 203.059 78.7419) (end 203.059 81.889) (width 0.2) (layer "B.Cu") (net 16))
 (segment (start 199.701 75.3839) (end 203.059 78.7419) (width 0.2) (layer "B.Cu") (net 16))
 (segment (start 203.059 81.889) (end 204.21 83.04) (width 0.2) (layer "B.Cu") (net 16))
 (segment (start 199.701 67.551) (end 199.701 75.3839) (width 0.2) (layer "B.Cu") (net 16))
 (segment (start 198.5 66.35) (end 199.701 67.551) (width 0.2) (layer "B.Cu") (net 16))
 (segment (start 218 84.13) (end 216.91 83.04) (width 0.2) (layer "B.Cu") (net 9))
 (segment (start 223.5 96.85) (end 218 91.35) (width 0.2) (layer "B.Cu") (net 9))
 (segment (start 218 91.35) (end 218 84.13) (width 0.2) (layer "B.Cu") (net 9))
 (segment (start 178.1 64.25) (end 200.098 64.25) (width 0.2) (layer "B.Cu") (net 20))
 (segment (start 202.299 71.598877) (end 208.950123 78.25) (width 0.2) (layer "B.Cu") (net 20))
 (segment (start 200.098 64.25) (end 202.299 66.451) (width 0.2) (layer "B.Cu") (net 20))
 (segment (start 173.5 68.85) (end 178.1 64.25) (width 0.2) (layer "B.Cu") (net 20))
 (segment (start 212.12 78.25) (end 214.37 80.5) (width 0.2) (layer "B.Cu") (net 20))
 (segment (start 202.299 66.451) (end 202.299 71.598877) (width 0.2) (layer "B.Cu") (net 20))
 (segment (start 208.950123 78.25) (end 212.12 78.25) (width 0.2) (layer "B.Cu") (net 20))
 (segment (start 173.5 94.35) (end 177.85 90) (width 0.2) (layer "F.Cu") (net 19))
 (segment (start 202.33 90) (end 209.29 83.04) (width 0.2) (layer "F.Cu") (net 19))
 (segment (start 177.85 90) (end 202.33 90) (width 0.2) (layer "F.Cu") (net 19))
 (segment (start 198.5 94.35) (end 203.06 94.35) (width 0.2) (layer "B.Cu") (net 5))
 (segment (start 203.06 94.35) (end 214.37 83.04) (width 0.2) (layer "B.Cu") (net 5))
 (segment (start 238.25 67.9875) (end 236.7 66.4375) (width 0.2) (layer "F.Cu") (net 23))
 (segment (start 237 94.4375) (end 237 91.75) (width 0.2) (layer "F.Cu") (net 23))
 (segment (start 235 63) (end 236.7 64.7) (width 0.2) (layer "F.Cu") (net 23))
 (segment (start 236.5 91.25) (end 232.75 91.25) (width 0.2) (layer "F.Cu") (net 23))
 (segment (start 228.5 80.5) (end 238.25 70.75) (width 0.2) (layer "F.Cu") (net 23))
 (segment (start 196.75 91.25) (end 190.1875 91.25) (width 0.2) (layer "F.Cu") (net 23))
 (segment (start 187 66.4375) (end 187.5625 66.4375) (width 0.2) (layer "F.Cu") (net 23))
 (segment (start 190.1875 91.25) (end 187 94.4375) (width 0.2) (layer "F.Cu") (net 23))
 (segment (start 224.53 80.5) (end 228.5 80.5) (width 0.2) (layer "F.Cu") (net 23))
 (segment (start 212 91.25) (end 196.75 91.25) (width 0.2) (layer "F.Cu") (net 23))
 (segment (start 232.75 91.25) (end 212 91.25) (width 0.2) (layer "F.Cu") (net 23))
 (segment (start 212 63) (end 235 63) (width 0.2) (layer "F.Cu") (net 23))
 (segment (start 236.7 64.7) (end 236.7 66.4375) (width 0.2) (layer "F.Cu") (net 23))
 (segment (start 232.74 91.25) (end 232.75 91.25) (width 0.2) (layer "F.Cu") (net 23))
 (segment (start 191 63) (end 212 63) (width 0.2) (layer "F.Cu") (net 23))
 (segment (start 187.5625 66.4375) (end 191 63) (width 0.2) (layer "F.Cu") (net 23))
 (segment (start 212 63) (end 212 66.4375) (width 0.2) (layer "F.Cu") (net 23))
 (segment (start 238.25 70.75) (end 238.25 67.9875) (width 0.2) (layer "F.Cu") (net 23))
 (segment (start 212 91.25) (end 212 94.4375) (width 0.2) (layer "F.Cu") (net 23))
 (segment (start 224.53 83.04) (end 232.74 91.25) (width 0.2) (layer "F.Cu") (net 23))
 (segment (start 237 91.75) (end 236.5 91.25) (width 0.2) (layer "F.Cu") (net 23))
 (segment (start 224.53 80.5) (end 224.53 83.04) (width 0.2) (layer "F.Cu") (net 23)))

